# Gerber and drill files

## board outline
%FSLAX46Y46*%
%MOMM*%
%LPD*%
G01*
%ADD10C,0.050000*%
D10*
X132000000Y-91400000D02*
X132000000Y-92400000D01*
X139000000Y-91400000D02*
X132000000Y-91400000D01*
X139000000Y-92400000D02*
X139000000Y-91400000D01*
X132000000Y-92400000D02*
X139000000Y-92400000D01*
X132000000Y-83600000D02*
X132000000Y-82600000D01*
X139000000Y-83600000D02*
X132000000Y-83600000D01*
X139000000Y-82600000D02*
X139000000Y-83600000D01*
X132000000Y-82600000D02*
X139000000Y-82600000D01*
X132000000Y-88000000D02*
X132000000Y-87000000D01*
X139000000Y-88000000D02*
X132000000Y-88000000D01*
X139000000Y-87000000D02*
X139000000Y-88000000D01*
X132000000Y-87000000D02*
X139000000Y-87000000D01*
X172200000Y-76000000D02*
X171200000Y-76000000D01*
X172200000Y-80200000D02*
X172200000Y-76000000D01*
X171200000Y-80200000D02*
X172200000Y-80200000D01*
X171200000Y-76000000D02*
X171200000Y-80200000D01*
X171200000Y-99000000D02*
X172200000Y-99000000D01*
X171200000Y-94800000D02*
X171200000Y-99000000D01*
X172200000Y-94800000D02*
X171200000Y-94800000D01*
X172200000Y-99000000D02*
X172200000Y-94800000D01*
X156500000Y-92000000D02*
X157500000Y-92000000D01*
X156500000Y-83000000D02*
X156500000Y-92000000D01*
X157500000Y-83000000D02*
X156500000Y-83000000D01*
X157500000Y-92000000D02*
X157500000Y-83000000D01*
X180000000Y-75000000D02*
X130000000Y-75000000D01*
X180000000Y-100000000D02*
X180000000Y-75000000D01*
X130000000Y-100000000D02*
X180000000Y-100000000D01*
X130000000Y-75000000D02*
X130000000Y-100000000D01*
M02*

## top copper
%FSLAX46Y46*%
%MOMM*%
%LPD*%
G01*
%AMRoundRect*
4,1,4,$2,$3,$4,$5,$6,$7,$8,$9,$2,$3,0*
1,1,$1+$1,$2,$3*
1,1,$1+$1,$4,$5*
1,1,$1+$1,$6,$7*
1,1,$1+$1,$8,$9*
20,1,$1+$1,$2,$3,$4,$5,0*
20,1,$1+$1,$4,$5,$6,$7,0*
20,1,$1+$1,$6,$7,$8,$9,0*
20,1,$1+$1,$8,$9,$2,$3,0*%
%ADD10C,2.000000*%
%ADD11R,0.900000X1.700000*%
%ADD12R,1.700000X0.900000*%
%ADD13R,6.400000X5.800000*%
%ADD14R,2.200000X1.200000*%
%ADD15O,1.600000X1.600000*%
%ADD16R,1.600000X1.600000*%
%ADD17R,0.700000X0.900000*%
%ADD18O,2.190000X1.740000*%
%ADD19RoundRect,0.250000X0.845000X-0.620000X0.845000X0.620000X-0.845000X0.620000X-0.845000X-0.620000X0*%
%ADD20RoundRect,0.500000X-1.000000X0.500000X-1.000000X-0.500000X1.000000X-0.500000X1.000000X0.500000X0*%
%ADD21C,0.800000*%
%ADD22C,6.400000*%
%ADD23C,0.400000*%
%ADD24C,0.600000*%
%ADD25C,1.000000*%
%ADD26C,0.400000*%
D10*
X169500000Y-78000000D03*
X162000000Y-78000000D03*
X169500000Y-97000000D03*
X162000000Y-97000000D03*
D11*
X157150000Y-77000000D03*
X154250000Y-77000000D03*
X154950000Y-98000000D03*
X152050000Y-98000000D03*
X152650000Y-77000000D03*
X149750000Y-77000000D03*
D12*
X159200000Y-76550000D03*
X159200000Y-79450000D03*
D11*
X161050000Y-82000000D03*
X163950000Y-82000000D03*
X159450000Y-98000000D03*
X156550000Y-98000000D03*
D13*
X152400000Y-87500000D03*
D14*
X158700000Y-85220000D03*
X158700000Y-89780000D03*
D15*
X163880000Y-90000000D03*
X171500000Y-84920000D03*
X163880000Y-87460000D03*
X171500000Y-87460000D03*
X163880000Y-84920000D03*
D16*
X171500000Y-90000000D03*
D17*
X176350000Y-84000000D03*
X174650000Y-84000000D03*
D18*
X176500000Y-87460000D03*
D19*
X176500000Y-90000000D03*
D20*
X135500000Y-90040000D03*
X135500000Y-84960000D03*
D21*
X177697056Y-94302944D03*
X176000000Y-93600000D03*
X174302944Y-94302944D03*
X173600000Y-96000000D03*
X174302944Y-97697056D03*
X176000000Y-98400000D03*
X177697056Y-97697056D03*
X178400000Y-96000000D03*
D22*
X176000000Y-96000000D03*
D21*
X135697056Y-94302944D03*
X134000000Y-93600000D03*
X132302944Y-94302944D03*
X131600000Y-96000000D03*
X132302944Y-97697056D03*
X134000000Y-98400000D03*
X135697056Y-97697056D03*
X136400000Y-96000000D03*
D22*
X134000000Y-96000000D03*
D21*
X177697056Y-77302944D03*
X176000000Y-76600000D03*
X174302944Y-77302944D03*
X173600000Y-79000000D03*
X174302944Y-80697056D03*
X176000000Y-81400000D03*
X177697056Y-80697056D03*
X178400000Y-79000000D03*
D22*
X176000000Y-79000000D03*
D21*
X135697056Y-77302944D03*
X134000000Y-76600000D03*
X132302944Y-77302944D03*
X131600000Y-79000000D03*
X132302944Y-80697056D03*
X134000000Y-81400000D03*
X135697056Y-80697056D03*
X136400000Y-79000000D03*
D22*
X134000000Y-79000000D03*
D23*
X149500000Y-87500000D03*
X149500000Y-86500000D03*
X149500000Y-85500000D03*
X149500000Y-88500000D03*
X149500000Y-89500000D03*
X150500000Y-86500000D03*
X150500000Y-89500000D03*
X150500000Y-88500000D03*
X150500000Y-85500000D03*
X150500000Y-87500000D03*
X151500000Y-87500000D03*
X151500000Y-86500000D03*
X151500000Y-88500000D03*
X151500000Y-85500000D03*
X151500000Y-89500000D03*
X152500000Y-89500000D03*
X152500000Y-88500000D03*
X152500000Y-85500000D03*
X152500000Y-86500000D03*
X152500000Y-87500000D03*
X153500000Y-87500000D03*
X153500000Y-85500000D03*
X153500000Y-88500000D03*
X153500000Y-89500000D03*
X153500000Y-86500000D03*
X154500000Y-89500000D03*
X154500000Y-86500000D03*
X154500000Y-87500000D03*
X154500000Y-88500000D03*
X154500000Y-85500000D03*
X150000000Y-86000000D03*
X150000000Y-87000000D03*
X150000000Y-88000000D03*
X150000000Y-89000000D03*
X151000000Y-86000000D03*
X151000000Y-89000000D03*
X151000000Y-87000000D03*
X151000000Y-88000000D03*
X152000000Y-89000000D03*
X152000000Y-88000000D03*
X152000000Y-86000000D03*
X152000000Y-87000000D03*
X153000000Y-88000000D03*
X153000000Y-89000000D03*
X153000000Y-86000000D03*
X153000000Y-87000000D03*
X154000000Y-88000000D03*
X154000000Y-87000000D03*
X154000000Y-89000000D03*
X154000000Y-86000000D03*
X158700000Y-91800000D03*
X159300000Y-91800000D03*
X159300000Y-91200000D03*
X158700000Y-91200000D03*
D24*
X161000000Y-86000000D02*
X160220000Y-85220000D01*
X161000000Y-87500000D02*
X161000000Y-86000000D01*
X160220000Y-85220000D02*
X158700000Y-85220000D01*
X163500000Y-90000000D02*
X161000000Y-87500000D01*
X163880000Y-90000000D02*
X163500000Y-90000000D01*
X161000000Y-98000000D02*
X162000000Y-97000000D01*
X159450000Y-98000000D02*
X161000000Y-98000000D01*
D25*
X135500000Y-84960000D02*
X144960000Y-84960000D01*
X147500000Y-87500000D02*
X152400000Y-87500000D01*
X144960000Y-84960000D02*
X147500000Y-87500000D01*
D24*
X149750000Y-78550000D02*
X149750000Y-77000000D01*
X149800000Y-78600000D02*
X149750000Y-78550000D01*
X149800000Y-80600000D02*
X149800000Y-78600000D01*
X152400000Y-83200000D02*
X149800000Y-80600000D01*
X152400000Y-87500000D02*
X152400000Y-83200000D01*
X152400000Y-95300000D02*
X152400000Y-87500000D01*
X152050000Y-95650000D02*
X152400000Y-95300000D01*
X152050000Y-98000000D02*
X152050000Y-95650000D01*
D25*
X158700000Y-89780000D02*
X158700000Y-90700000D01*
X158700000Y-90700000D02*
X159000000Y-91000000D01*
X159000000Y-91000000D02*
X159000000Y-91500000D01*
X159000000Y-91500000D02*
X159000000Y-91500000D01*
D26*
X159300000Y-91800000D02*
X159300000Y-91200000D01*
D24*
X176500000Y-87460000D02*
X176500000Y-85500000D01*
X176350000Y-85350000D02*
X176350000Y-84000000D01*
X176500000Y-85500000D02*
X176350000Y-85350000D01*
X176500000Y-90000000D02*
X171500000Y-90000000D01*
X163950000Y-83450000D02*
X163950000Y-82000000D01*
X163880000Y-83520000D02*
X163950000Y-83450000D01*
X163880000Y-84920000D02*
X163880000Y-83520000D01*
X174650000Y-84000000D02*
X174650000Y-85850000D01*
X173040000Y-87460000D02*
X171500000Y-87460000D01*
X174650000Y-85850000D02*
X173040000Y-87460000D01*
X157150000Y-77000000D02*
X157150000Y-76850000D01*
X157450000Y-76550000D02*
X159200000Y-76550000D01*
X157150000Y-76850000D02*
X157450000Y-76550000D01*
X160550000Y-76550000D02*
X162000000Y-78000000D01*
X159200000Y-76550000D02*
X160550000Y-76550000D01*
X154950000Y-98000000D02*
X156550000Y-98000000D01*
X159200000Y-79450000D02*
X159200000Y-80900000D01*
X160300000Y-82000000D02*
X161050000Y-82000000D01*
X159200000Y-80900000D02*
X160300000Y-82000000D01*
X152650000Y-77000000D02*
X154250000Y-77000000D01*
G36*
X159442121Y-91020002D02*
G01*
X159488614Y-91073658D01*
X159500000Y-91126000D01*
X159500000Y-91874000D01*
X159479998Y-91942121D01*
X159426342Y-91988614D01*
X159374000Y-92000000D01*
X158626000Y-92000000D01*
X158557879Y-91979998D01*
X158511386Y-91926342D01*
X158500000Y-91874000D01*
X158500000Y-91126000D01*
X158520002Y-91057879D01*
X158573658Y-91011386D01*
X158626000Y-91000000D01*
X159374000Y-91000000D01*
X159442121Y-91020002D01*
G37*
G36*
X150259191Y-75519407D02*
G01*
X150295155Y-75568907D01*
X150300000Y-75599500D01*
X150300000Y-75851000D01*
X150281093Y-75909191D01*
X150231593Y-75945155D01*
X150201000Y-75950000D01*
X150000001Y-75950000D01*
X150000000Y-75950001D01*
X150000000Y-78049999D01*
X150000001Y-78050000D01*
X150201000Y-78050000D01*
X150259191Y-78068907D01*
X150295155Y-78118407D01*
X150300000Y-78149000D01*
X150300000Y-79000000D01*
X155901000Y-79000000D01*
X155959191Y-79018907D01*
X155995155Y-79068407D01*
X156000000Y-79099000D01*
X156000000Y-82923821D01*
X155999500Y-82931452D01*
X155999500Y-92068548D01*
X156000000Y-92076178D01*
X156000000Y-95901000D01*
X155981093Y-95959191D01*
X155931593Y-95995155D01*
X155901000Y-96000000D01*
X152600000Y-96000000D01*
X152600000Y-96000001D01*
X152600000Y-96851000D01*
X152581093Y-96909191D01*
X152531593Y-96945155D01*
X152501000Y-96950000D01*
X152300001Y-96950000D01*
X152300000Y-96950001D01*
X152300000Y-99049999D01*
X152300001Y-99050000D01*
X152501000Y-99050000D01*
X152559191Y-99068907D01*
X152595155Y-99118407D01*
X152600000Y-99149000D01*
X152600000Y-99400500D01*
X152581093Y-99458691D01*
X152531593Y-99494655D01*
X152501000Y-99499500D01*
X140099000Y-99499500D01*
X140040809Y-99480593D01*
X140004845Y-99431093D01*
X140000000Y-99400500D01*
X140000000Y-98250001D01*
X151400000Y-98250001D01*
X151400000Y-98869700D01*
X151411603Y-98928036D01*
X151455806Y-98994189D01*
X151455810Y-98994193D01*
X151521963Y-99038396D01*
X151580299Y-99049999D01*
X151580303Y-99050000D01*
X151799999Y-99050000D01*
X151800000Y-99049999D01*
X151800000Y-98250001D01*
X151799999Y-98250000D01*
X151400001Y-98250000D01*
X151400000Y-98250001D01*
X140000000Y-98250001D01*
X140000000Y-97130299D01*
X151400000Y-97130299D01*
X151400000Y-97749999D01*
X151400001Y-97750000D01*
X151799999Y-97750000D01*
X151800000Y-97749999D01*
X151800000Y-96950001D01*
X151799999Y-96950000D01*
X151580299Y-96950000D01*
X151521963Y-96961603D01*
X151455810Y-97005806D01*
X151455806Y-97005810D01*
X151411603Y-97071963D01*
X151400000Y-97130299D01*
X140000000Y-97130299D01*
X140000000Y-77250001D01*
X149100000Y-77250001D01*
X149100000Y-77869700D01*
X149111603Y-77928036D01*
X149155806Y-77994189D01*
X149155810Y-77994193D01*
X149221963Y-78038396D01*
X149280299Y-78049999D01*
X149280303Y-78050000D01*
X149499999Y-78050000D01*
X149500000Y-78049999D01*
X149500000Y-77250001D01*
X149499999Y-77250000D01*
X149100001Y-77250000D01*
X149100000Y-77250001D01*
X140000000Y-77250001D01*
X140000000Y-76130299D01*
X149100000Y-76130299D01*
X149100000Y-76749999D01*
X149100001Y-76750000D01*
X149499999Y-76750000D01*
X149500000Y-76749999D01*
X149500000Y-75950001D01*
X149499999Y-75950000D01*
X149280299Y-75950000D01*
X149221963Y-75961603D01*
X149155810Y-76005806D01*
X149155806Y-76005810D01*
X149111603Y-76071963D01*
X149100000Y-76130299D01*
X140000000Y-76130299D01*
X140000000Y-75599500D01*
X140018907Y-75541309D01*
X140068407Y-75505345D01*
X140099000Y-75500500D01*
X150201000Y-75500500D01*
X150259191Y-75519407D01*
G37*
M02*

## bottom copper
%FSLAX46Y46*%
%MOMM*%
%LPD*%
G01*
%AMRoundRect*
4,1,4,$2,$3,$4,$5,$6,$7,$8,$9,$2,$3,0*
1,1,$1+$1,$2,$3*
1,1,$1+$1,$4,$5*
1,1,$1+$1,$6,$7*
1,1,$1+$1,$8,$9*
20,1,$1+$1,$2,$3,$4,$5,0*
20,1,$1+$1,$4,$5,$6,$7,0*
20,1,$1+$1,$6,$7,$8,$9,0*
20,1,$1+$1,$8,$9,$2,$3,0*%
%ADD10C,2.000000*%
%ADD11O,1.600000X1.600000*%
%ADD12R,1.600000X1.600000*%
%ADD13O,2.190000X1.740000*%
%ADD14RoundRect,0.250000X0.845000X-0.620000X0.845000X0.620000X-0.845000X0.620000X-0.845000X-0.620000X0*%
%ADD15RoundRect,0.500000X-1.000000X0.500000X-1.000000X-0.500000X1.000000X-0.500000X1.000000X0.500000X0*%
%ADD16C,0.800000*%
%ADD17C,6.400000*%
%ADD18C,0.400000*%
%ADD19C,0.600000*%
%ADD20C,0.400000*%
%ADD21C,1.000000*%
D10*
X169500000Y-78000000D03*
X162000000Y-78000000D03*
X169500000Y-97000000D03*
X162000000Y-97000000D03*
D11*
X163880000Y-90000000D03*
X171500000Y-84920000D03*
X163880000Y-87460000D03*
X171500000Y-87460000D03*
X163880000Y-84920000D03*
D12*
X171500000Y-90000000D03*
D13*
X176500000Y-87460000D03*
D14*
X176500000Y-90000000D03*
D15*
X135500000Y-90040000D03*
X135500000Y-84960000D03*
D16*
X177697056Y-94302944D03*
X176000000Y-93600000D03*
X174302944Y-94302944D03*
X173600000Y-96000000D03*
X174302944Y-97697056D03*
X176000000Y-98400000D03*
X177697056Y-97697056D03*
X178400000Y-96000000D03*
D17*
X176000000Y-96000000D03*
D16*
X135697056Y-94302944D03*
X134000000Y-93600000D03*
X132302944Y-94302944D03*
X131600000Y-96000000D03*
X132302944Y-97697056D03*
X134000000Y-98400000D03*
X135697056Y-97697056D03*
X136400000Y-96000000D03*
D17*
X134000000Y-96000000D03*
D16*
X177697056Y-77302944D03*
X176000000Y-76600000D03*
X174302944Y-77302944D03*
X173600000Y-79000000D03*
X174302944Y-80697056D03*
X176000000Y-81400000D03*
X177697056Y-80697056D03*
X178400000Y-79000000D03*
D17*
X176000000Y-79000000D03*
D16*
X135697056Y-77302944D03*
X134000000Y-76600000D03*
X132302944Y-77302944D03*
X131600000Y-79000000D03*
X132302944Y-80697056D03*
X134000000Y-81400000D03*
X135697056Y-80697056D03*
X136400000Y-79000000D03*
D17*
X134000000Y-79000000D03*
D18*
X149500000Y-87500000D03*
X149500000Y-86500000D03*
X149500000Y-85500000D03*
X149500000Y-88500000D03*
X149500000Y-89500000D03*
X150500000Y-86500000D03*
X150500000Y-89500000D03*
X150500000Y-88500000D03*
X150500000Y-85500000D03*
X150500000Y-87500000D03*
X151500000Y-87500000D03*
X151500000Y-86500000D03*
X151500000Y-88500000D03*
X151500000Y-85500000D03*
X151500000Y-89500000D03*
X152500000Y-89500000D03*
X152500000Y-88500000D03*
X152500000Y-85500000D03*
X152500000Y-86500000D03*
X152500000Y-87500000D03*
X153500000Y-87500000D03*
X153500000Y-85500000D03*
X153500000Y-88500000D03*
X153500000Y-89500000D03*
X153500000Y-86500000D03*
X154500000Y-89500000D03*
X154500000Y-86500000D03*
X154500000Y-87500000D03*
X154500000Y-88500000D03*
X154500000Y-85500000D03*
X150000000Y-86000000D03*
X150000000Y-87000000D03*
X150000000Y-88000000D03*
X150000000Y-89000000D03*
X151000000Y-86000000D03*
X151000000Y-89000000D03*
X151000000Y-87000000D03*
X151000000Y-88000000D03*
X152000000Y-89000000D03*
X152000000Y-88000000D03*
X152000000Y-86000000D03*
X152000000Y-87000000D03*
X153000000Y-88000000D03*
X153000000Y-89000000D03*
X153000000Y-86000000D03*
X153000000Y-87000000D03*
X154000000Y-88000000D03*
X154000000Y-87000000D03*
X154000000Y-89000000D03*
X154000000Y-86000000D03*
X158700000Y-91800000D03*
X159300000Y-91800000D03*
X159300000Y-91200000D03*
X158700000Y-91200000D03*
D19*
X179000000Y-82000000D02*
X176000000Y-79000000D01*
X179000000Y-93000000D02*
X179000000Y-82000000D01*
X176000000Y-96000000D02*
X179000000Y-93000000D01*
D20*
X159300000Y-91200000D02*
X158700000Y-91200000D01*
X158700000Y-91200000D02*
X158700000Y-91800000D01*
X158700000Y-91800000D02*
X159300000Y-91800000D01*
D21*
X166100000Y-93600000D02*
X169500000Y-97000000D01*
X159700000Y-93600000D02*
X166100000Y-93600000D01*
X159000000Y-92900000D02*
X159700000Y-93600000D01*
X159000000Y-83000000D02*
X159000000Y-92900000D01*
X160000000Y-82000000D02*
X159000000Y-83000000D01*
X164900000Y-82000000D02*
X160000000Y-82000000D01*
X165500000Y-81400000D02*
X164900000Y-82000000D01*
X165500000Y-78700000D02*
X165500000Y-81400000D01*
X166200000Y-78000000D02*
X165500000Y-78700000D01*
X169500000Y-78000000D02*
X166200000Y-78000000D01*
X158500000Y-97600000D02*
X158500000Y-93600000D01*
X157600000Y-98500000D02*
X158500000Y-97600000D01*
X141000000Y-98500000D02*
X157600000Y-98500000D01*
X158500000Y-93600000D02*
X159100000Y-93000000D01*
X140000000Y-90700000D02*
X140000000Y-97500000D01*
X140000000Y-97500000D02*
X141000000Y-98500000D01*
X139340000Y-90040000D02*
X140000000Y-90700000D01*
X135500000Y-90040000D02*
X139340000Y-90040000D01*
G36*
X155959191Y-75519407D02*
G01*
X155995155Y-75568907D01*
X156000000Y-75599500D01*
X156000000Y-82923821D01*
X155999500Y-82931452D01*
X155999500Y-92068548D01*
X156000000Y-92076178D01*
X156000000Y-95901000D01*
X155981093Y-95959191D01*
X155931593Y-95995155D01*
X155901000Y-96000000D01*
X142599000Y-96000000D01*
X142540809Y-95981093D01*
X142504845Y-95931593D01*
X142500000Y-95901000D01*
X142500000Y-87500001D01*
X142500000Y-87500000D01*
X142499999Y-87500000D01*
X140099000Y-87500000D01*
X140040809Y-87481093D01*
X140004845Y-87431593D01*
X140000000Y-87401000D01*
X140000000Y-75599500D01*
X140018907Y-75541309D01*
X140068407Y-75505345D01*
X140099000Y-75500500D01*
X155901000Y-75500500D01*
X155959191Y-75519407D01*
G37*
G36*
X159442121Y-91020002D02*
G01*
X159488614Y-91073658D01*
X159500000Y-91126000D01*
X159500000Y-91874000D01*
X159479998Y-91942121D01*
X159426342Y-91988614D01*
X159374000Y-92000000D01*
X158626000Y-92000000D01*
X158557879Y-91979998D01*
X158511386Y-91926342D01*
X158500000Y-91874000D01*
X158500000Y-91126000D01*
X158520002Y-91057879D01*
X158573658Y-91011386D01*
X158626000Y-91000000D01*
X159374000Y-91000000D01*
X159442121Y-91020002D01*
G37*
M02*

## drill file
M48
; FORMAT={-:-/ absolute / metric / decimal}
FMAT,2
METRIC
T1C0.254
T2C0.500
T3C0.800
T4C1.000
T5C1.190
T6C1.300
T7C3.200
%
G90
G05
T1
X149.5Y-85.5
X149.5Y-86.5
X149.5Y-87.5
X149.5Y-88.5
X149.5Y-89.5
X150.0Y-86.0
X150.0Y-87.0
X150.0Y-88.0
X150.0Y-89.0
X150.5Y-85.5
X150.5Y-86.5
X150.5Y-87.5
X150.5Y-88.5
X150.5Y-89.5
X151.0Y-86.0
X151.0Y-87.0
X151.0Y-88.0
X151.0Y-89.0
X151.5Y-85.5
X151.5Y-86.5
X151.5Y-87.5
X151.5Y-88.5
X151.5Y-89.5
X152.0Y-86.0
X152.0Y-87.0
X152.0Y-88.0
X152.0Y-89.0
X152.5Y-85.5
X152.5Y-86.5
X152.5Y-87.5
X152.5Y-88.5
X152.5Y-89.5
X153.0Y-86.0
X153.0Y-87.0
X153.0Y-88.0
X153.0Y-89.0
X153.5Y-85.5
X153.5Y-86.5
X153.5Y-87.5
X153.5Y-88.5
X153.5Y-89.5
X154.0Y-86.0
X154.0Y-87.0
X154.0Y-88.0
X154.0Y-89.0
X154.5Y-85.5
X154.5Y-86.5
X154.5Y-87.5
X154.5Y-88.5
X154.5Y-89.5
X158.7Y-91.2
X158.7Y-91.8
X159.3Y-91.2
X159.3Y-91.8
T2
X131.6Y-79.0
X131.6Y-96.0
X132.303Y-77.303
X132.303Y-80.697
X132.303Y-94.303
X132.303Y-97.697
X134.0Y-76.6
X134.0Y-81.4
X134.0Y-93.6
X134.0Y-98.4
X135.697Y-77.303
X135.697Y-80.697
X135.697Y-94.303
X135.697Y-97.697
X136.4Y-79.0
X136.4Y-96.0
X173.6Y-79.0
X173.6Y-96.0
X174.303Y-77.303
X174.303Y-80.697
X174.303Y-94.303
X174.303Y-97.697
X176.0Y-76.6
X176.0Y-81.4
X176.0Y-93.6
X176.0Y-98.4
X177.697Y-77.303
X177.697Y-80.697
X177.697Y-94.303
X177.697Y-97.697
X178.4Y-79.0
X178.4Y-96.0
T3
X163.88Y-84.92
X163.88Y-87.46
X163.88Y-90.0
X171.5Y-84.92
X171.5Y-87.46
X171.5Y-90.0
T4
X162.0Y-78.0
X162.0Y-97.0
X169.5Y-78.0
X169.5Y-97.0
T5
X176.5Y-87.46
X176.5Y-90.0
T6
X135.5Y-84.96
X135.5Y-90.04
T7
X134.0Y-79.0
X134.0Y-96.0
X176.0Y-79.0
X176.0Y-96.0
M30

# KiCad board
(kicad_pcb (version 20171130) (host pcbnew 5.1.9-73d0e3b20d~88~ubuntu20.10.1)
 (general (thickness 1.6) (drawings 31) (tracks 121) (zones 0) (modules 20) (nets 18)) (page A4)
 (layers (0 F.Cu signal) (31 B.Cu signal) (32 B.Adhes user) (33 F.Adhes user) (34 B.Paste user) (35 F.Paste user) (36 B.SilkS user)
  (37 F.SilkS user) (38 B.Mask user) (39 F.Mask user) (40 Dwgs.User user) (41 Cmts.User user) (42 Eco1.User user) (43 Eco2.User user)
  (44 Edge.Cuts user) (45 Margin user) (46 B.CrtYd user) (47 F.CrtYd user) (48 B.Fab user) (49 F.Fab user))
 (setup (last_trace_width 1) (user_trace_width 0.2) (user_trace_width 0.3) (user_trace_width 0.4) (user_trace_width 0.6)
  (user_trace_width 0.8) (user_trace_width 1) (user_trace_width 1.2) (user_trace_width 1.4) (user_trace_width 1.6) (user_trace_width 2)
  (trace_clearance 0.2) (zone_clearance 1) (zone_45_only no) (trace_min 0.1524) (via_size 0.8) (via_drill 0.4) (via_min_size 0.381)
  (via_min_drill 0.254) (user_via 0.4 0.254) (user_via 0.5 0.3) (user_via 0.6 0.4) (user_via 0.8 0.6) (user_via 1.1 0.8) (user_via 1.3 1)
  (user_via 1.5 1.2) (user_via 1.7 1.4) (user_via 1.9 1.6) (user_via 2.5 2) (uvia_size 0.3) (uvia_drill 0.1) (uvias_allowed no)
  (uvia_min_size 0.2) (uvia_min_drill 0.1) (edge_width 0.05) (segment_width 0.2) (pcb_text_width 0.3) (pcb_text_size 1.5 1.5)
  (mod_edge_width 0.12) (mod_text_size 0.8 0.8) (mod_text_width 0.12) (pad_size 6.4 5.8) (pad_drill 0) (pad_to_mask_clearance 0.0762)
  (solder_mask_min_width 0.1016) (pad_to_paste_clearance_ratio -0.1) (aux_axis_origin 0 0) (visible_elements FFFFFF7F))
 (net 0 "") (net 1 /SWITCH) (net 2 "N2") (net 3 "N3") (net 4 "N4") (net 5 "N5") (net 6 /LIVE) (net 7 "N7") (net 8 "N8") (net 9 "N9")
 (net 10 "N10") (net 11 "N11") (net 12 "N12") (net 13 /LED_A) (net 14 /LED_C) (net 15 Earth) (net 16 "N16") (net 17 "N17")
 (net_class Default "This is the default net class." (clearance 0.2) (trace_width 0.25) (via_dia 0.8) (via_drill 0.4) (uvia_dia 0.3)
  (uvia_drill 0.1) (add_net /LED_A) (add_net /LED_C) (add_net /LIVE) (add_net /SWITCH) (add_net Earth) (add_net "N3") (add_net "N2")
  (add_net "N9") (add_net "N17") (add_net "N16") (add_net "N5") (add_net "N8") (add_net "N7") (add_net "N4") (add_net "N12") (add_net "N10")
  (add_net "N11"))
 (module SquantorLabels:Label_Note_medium (layer F.Cu) (at 145.3 87.4 90)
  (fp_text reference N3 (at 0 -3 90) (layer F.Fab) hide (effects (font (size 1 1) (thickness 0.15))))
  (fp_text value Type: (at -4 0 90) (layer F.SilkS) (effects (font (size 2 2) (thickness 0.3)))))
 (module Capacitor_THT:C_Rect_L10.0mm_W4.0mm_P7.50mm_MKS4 (layer F.Cu) (at 162 78)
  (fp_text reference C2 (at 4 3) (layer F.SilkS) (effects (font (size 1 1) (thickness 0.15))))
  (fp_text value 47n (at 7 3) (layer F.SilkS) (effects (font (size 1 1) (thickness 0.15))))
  (pad 2 thru_hole circle (at 7.5 0) (size 2 2) (drill 1) (layers *.Cu *.Mask) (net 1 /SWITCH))
  (pad 1 thru_hole circle (at 0 0) (size 2 2) (drill 1) (layers *.Cu *.Mask) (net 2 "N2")))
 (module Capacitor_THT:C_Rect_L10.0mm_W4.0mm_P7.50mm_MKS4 (layer F.Cu) (at 162 97)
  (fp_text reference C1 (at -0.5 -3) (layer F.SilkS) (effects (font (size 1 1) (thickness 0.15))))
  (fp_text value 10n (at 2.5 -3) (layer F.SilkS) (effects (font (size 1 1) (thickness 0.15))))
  (pad 2 thru_hole circle (at 7.5 0) (size 2 2) (drill 1) (layers *.Cu *.Mask) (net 1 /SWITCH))
  (pad 1 thru_hole circle (at 0 0) (size 2 2) (drill 1) (layers *.Cu *.Mask) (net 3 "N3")))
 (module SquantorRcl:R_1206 (layer F.Cu) (at 155.7 77)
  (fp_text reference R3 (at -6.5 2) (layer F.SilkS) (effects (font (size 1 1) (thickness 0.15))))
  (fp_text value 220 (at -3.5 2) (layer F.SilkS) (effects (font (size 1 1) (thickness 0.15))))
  (pad 2 smd rect (at 1.45 0) (size 0.9 1.7) (layers F.Cu F.Paste F.Mask) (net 2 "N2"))
  (pad 1 smd rect (at -1.45 0) (size 0.9 1.7) (layers F.Cu F.Paste F.Mask) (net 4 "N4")))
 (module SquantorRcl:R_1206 (layer F.Cu) (at 153.5 98)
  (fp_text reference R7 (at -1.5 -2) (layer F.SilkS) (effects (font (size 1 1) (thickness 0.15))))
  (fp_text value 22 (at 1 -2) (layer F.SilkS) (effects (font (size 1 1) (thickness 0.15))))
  (pad 2 smd rect (at 1.45 0) (size 0.9 1.7) (layers F.Cu F.Paste F.Mask) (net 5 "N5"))
  (pad 1 smd rect (at -1.45 0) (size 0.9 1.7) (layers F.Cu F.Paste F.Mask) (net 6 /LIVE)))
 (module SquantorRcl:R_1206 (layer F.Cu) (at 151.2 77)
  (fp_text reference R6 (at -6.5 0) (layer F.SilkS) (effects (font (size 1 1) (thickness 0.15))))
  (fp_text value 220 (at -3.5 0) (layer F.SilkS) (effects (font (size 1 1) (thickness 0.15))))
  (pad 2 smd rect (at 1.45 0) (size 0.9 1.7) (layers F.Cu F.Paste F.Mask) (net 4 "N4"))
  (pad 1 smd rect (at -1.45 0) (size 0.9 1.7) (layers F.Cu F.Paste F.Mask) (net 6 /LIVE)))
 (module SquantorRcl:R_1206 (layer F.Cu) (at 159.2 78 90)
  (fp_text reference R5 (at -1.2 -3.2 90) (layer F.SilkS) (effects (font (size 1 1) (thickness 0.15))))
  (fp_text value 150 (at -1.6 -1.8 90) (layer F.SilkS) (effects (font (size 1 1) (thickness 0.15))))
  (pad 2 smd rect (at 1.45 0 90) (size 0.9 1.7) (layers F.Cu F.Paste F.Mask) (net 2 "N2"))
  (pad 1 smd rect (at -1.45 0 90) (size 0.9 1.7) (layers F.Cu F.Paste F.Mask) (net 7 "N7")))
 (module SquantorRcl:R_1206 (layer F.Cu) (at 162.5 82 180)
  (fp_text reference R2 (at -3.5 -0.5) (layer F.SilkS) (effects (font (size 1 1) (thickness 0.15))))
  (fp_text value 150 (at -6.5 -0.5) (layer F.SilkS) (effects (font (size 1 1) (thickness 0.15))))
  (pad 2 smd rect (at 1.45 0 180) (size 0.9 1.7) (layers F.Cu F.Paste F.Mask) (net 7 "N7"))
  (pad 1 smd rect (at -1.45 0 180) (size 0.9 1.7) (layers F.Cu F.Paste F.Mask) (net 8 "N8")))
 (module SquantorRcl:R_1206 (layer F.Cu) (at 158 98)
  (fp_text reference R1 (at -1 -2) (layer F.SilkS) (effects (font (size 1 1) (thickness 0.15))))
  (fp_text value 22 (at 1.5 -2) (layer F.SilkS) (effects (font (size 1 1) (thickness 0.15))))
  (pad 2 smd rect (at 1.45 0) (size 0.9 1.7) (layers F.Cu F.Paste F.Mask) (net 3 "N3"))
  (pad 1 smd rect (at -1.45 0) (size 0.9 1.7) (layers F.Cu F.Paste F.Mask) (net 5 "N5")))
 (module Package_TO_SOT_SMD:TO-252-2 (layer F.Cu) (at 154.5 87.5 180)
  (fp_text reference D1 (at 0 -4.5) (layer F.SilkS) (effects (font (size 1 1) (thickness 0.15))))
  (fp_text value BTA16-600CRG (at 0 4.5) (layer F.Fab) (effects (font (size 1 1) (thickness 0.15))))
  (pad "" smd rect (at 0.425 1.525 180) (size 3.05 2.75) (layers F.Paste))
  (pad "" smd rect (at 3.775 -1.525 180) (size 3.05 2.75) (layers F.Paste))
  (pad "" smd rect (at 0.425 -1.525 180) (size 3.05 2.75) (layers F.Paste))
  (pad "" smd rect (at 3.775 1.525 180) (size 3.05 2.75) (layers F.Paste))
  (pad 2 smd rect (at 2.1 0 180) (size 6.4 5.8) (layers F.Cu F.Mask) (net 6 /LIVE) (zone_connect 2))
  (pad 3 smd rect (at -4.2 2.28 180) (size 2.2 1.2) (layers F.Cu F.Paste F.Mask) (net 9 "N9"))
  (pad 1 smd rect (at -4.2 -2.28 180) (size 2.2 1.2) (layers F.Cu F.Paste F.Mask) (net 1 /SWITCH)))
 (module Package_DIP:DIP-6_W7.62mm (layer F.Cu) (at 171.5 90 180)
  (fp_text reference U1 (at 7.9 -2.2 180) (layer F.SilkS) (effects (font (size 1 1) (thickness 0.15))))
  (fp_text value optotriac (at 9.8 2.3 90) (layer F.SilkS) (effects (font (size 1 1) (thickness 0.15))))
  (pad 6 thru_hole oval (at 7.62 0 180) (size 1.6 1.6) (drill 0.8) (layers *.Cu *.Mask) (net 9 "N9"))
  (pad 3 thru_hole oval (at 0 5.08 180) (size 1.6 1.6) (drill 0.8) (layers *.Cu *.Mask) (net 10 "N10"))
  (pad 5 thru_hole oval (at 7.62 2.54 180) (size 1.6 1.6) (drill 0.8) (layers *.Cu *.Mask) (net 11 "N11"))
  (pad 2 thru_hole oval (at 0 2.54 180) (size 1.6 1.6) (drill 0.8) (layers *.Cu *.Mask) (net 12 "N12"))
  (pad 4 thru_hole oval (at 7.62 5.08 180) (size 1.6 1.6) (drill 0.8) (layers *.Cu *.Mask) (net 8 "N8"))
  (pad 1 thru_hole rect (at 0 0 180) (size 1.6 1.6) (drill 0.8) (layers *.Cu *.Mask) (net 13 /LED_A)))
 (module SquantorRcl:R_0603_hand (layer F.Cu) (at 175.5 84)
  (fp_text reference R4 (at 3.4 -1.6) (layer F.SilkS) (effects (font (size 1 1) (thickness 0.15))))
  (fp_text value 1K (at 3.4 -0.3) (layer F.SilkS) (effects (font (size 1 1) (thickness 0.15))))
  (pad 2 smd rect (at 0.85 0) (size 0.7 0.9) (layers F.Cu F.Paste F.Mask) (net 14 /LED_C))
  (pad 1 smd rect (at -0.85 0) (size 0.7 0.9) (layers F.Cu F.Paste F.Mask) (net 12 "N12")))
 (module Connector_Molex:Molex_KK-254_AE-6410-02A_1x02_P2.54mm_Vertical (layer F.Cu) (at 176.5 90 90)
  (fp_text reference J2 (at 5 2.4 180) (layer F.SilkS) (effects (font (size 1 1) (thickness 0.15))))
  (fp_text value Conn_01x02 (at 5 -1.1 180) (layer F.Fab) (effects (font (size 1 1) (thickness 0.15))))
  (pad 2 thru_hole oval (at 2.54 0 90) (size 1.74 2.19) (drill 1.19) (layers *.Cu *.Mask) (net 14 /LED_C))
  (pad 1 thru_hole roundrect (at 0 0 90) (size 1.74 2.19) (drill 1.19) (layers *.Cu *.Mask) (roundrect_rratio 0.143678) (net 13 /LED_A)))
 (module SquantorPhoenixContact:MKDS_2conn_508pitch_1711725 (layer F.Cu) (at 135.5 87.5 270)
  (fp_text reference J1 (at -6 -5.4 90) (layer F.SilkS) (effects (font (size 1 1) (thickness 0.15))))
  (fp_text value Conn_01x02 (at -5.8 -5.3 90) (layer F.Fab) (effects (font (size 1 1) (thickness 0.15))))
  (pad 2 thru_hole roundrect (at 2.54 0 270) (size 2 3) (drill 1.3) (layers *.Cu *.Mask) (roundrect_rratio 0.25) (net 1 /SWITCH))
  (pad 1 thru_hole roundrect (at -2.54 0 270) (size 2 3) (drill 1.3) (layers *.Cu *.Mask) (roundrect_rratio 0.25) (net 6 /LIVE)))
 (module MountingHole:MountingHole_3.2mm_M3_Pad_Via (layer F.Cu) (at 176 96)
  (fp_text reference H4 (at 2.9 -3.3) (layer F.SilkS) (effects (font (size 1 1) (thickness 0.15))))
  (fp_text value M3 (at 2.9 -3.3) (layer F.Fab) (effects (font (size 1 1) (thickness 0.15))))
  (pad 1 thru_hole circle (at 1.697056 -1.697056) (size 0.8 0.8) (drill 0.5) (layers *.Cu *.Mask) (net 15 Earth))
  (pad 1 thru_hole circle (at 0 -2.4) (size 0.8 0.8) (drill 0.5) (layers *.Cu *.Mask) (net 15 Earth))
  (pad 1 thru_hole circle (at -1.697056 -1.697056) (size 0.8 0.8) (drill 0.5) (layers *.Cu *.Mask) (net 15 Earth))
  (pad 1 thru_hole circle (at -2.4 0) (size 0.8 0.8) (drill 0.5) (layers *.Cu *.Mask) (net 15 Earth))
  (pad 1 thru_hole circle (at -1.697056 1.697056) (size 0.8 0.8) (drill 0.5) (layers *.Cu *.Mask) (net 15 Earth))
  (pad 1 thru_hole circle (at 0 2.4) (size 0.8 0.8) (drill 0.5) (layers *.Cu *.Mask) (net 15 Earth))
  (pad 1 thru_hole circle (at 1.697056 1.697056) (size 0.8 0.8) (drill 0.5) (layers *.Cu *.Mask) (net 15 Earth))
  (pad 1 thru_hole circle (at 2.4 0) (size 0.8 0.8) (drill 0.5) (layers *.Cu *.Mask) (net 15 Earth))
  (pad 1 thru_hole circle (at 0 0) (size 6.4 6.4) (drill 3.2) (layers *.Cu *.Mask) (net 15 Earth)))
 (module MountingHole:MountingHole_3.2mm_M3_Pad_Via (layer F.Cu) (at 134 96)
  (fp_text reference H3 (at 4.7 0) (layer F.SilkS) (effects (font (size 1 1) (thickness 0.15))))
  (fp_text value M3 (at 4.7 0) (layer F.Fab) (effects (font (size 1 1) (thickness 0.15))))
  (pad 1 thru_hole circle (at 1.697056 -1.697056) (size 0.8 0.8) (drill 0.5) (layers *.Cu *.Mask) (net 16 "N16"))
  (pad 1 thru_hole circle (at 0 -2.4) (size 0.8 0.8) (drill 0.5) (layers *.Cu *.Mask) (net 16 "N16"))
  (pad 1 thru_hole circle (at -1.697056 -1.697056) (size 0.8 0.8) (drill 0.5) (layers *.Cu *.Mask) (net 16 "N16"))
  (pad 1 thru_hole circle (at -2.4 0) (size 0.8 0.8) (drill 0.5) (layers *.Cu *.Mask) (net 16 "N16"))
  (pad 1 thru_hole circle (at -1.697056 1.697056) (size 0.8 0.8) (drill 0.5) (layers *.Cu *.Mask) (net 16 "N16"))
  (pad 1 thru_hole circle (at 0 2.4) (size 0.8 0.8) (drill 0.5) (layers *.Cu *.Mask) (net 16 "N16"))
  (pad 1 thru_hole circle (at 1.697056 1.697056) (size 0.8 0.8) (drill 0.5) (layers *.Cu *.Mask) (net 16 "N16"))
  (pad 1 thru_hole circle (at 2.4 0) (size 0.8 0.8) (drill 0.5) (layers *.Cu *.Mask) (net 16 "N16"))
  (pad 1 thru_hole circle (at 0 0) (size 6.4 6.4) (drill 3.2) (layers *.Cu *.Mask) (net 16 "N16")))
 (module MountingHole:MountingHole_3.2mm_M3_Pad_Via (layer F.Cu) (at 176 79)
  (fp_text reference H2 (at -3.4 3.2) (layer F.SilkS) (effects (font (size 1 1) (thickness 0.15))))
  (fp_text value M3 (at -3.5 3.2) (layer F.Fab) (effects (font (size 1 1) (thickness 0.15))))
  (pad 1 thru_hole circle (at 1.697056 -1.697056) (size 0.8 0.8) (drill 0.5) (layers *.Cu *.Mask) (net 15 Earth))
  (pad 1 thru_hole circle (at 0 -2.4) (size 0.8 0.8) (drill 0.5) (layers *.Cu *.Mask) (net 15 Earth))
  (pad 1 thru_hole circle (at -1.697056 -1.697056) (size 0.8 0.8) (drill 0.5) (layers *.Cu *.Mask) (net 15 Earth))
  (pad 1 thru_hole circle (at -2.4 0) (size 0.8 0.8) (drill 0.5) (layers *.Cu *.Mask) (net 15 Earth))
  (pad 1 thru_hole circle (at -1.697056 1.697056) (size 0.8 0.8) (drill 0.5) (layers *.Cu *.Mask) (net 15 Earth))
  (pad 1 thru_hole circle (at 0 2.4) (size 0.8 0.8) (drill 0.5) (layers *.Cu *.Mask) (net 15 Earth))
  (pad 1 thru_hole circle (at 1.697056 1.697056) (size 0.8 0.8) (drill 0.5) (layers *.Cu *.Mask) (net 15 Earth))
  (pad 1 thru_hole circle (at 2.4 0) (size 0.8 0.8) (drill 0.5) (layers *.Cu *.Mask) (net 15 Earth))
  (pad 1 thru_hole circle (at 0 0) (size 6.4 6.4) (drill 3.2) (layers *.Cu *.Mask) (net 15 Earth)))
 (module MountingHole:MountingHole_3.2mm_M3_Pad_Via (layer F.Cu) (at 134 79)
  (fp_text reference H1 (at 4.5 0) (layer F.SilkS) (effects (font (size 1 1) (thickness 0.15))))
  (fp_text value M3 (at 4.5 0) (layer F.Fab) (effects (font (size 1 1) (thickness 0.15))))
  (pad 1 thru_hole circle (at 1.697056 -1.697056) (size 0.8 0.8) (drill 0.5) (layers *.Cu *.Mask) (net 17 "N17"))
  (pad 1 thru_hole circle (at 0 -2.4) (size 0.8 0.8) (drill 0.5) (layers *.Cu *.Mask) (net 17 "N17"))
  (pad 1 thru_hole circle (at -1.697056 -1.697056) (size 0.8 0.8) (drill 0.5) (layers *.Cu *.Mask) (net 17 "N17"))
  (pad 1 thru_hole circle (at -2.4 0) (size 0.8 0.8) (drill 0.5) (layers *.Cu *.Mask) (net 17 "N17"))
  (pad 1 thru_hole circle (at -1.697056 1.697056) (size 0.8 0.8) (drill 0.5) (layers *.Cu *.Mask) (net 17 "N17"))
  (pad 1 thru_hole circle (at 0 2.4) (size 0.8 0.8) (drill 0.5) (layers *.Cu *.Mask) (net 17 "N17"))
  (pad 1 thru_hole circle (at 1.697056 1.697056) (size 0.8 0.8) (drill 0.5) (layers *.Cu *.Mask) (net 17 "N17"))
  (pad 1 thru_hole circle (at 2.4 0) (size 0.8 0.8) (drill 0.5) (layers *.Cu *.Mask) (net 17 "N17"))
  (pad 1 thru_hole circle (at 0 0) (size 6.4 6.4) (drill 3.2) (layers *.Cu *.Mask) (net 17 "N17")))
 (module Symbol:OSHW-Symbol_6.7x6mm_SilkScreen (layer B.Cu) (at 143.6 87.5 270)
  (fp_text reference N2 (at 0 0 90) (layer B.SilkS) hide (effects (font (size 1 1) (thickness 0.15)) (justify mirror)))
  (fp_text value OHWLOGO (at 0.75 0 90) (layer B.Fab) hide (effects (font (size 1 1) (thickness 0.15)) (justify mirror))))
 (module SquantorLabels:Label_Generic (layer B.Cu) (at 147.5 86.9 270)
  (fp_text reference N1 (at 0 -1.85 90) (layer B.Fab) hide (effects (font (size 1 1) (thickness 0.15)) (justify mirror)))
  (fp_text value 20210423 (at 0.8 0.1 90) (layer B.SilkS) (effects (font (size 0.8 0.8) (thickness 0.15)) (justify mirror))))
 (gr_line (start 132 91.4) (end 132 92.4) (layer Edge.Cuts) (width 0.05))
 (gr_line (start 139 91.4) (end 132 91.4) (layer Edge.Cuts) (width 0.05))
 (gr_line (start 139 92.4) (end 139 91.4) (layer Edge.Cuts) (width 0.05))
 (gr_line (start 132 92.4) (end 139 92.4) (layer Edge.Cuts) (width 0.05))
 (gr_line (start 132 83.6) (end 132 82.6) (layer Edge.Cuts) (width 0.05))
 (gr_line (start 139 83.6) (end 132 83.6) (layer Edge.Cuts) (width 0.05))
 (gr_line (start 139 82.6) (end 139 83.6) (layer Edge.Cuts) (width 0.05))
 (gr_line (start 132 82.6) (end 139 82.6) (layer Edge.Cuts) (width 0.05))
 (gr_line (start 132 88) (end 132 87) (layer Edge.Cuts) (width 0.05))
 (gr_line (start 139 88) (end 132 88) (layer Edge.Cuts) (width 0.05))
 (gr_line (start 139 87) (end 139 88) (layer Edge.Cuts) (width 0.05))
 (gr_line (start 132 87) (end 139 87) (layer Edge.Cuts) (width 0.05))
 (gr_line (start 172.2 76) (end 171.2 76) (layer Edge.Cuts) (width 0.05))
 (gr_line (start 172.2 80.2) (end 172.2 76) (layer Edge.Cuts) (width 0.05))
 (gr_line (start 171.2 80.2) (end 172.2 80.2) (layer Edge.Cuts) (width 0.05))
 (gr_line (start 171.2 76) (end 171.2 80.2) (layer Edge.Cuts) (width 0.05))
 (gr_line (start 171.2 99) (end 172.2 99) (layer Edge.Cuts) (width 0.05))
 (gr_line (start 171.2 94.8) (end 171.2 99) (layer Edge.Cuts) (width 0.05))
 (gr_line (start 172.2 94.8) (end 171.2 94.8) (layer Edge.Cuts) (width 0.05))
 (gr_line (start 172.2 99) (end 172.2 94.8) (layer Edge.Cuts) (width 0.05))
 (gr_line (start 156.5 92) (end 157.5 92) (layer Edge.Cuts) (width 0.05))
 (gr_line (start 156.5 83) (end 156.5 92) (layer Edge.Cuts) (width 0.05))
 (gr_line (start 157.5 83) (end 156.5 83) (layer Edge.Cuts) (width 0.05))
 (gr_line (start 157.5 92) (end 157.5 83) (layer Edge.Cuts) (width 0.05))
 (gr_line (start 180 75) (end 130 75) (layer Edge.Cuts) (width 0.05))
 (gr_line (start 180 100) (end 180 75) (layer Edge.Cuts) (width 0.05))
 (gr_line (start 130 100) (end 180 100) (layer Edge.Cuts) (width 0.05))
 (gr_line (start 130 75) (end 130 100) (layer Edge.Cuts) (width 0.05))
 (segment (start 161 86) (end 160.22 85.22) (width 0.6) (layer F.Cu) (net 9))
 (segment (start 161 87.5) (end 161 86) (width 0.6) (layer F.Cu) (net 9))
 (segment (start 160.22 85.22) (end 158.7 85.22) (width 0.6) (layer F.Cu) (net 9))
 (segment (start 163.5 90) (end 161 87.5) (width 0.6) (layer F.Cu) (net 9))
 (segment (start 163.88 90) (end 163.5 90) (width 0.6) (layer F.Cu) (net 9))
 (segment (start 179 82) (end 176 79) (width 0.6) (layer B.Cu) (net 15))
 (segment (start 179 93) (end 179 82) (width 0.6) (layer B.Cu) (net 15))
 (segment (start 176 96) (end 179 93) (width 0.6) (layer B.Cu) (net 15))
 (segment (start 161 98) (end 162 97) (width 0.6) (layer F.Cu) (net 3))
 (segment (start 159.45 98) (end 161 98) (width 0.6) (layer F.Cu) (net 3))
 (segment (start 135.5 84.96) (end 144.96 84.96) (width 1) (layer F.Cu) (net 6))
 (segment (start 147.5 87.5) (end 152.4 87.5) (width 1) (layer F.Cu) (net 6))
 (segment (start 144.96 84.96) (end 147.5 87.5) (width 1) (layer F.Cu) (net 6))
 (via (at 149.5 87.5) (size 0.4) (drill 0.254) (layers F.Cu B.Cu) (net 6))
 (via (at 149.5 86.5) (size 0.4) (drill 0.254) (layers F.Cu B.Cu) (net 6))
 (via (at 149.5 85.5) (size 0.4) (drill 0.254) (layers F.Cu B.Cu) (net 6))
 (via (at 149.5 88.5) (size 0.4) (drill 0.254) (layers F.Cu B.Cu) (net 6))
 (via (at 149.5 89.5) (size 0.4) (drill 0.254) (layers F.Cu B.Cu) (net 6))
 (via (at 150.5 86.5) (size 0.4) (drill 0.254) (layers F.Cu B.Cu) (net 6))
 (via (at 150.5 89.5) (size 0.4) (drill 0.254) (layers F.Cu B.Cu) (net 6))
 (via (at 150.5 88.5) (size 0.4) (drill 0.254) (layers F.Cu B.Cu) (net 6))
 (via (at 150.5 85.5) (size 0.4) (drill 0.254) (layers F.Cu B.Cu) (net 6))
 (via (at 150.5 87.5) (size 0.4) (drill 0.254) (layers F.Cu B.Cu) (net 6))
 (via (at 151.5 87.5) (size 0.4) (drill 0.254) (layers F.Cu B.Cu) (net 6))
 (via (at 151.5 86.5) (size 0.4) (drill 0.254) (layers F.Cu B.Cu) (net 6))
 (via (at 151.5 88.5) (size 0.4) (drill 0.254) (layers F.Cu B.Cu) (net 6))
 (via (at 151.5 85.5) (size 0.4) (drill 0.254) (layers F.Cu B.Cu) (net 6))
 (via (at 151.5 89.5) (size 0.4) (drill 0.254) (layers F.Cu B.Cu) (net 6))
 (via (at 152.5 89.5) (size 0.4) (drill 0.254) (layers F.Cu B.Cu) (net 6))
 (via (at 152.5 88.5) (size 0.4) (drill 0.254) (layers F.Cu B.Cu) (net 6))
 (via (at 152.5 85.5) (size 0.4) (drill 0.254) (layers F.Cu B.Cu) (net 6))
 (via (at 152.5 86.5) (size 0.4) (drill 0.254) (layers F.Cu B.Cu) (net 6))
 (via (at 152.5 87.5) (size 0.4) (drill 0.254) (layers F.Cu B.Cu) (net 6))
 (via (at 153.5 87.5) (size 0.4) (drill 0.254) (layers F.Cu B.Cu) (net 6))
 (via (at 153.5 85.5) (size 0.4) (drill 0.254) (layers F.Cu B.Cu) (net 6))
 (via (at 153.5 88.5) (size 0.4) (drill 0.254) (layers F.Cu B.Cu) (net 6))
 (via (at 153.5 89.5) (size 0.4) (drill 0.254) (layers F.Cu B.Cu) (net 6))
 (via (at 153.5 86.5) (size 0.4) (drill 0.254) (layers F.Cu B.Cu) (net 6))
 (via (at 154.5 89.5) (size 0.4) (drill 0.254) (layers F.Cu B.Cu) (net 6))
 (via (at 154.5 86.5) (size 0.4) (drill 0.254) (layers F.Cu B.Cu) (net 6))
 (via (at 154.5 87.5) (size 0.4) (drill 0.254) (layers F.Cu B.Cu) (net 6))
 (via (at 154.5 88.5) (size 0.4) (drill 0.254) (layers F.Cu B.Cu) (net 6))
 (via (at 154.5 85.5) (size 0.4) (drill 0.254) (layers F.Cu B.Cu) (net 6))
 (via (at 150 86) (size 0.4) (drill 0.254) (layers F.Cu B.Cu) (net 6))
 (via (at 150 87) (size 0.4) (drill 0.254) (layers F.Cu B.Cu) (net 6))
 (via (at 150 88) (size 0.4) (drill 0.254) (layers F.Cu B.Cu) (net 6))
 (via (at 150 89) (size 0.4) (drill 0.254) (layers F.Cu B.Cu) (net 6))
 (via (at 151 86) (size 0.4) (drill 0.254) (layers F.Cu B.Cu) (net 6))
 (via (at 151 89) (size 0.4) (drill 0.254) (layers F.Cu B.Cu) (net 6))
 (via (at 151 87) (size 0.4) (drill 0.254) (layers F.Cu B.Cu) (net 6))
 (via (at 151 88) (size 0.4) (drill 0.254) (layers F.Cu B.Cu) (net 6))
 (via (at 152 89) (size 0.4) (drill 0.254) (layers F.Cu B.Cu) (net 6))
 (via (at 152 88) (size 0.4) (drill 0.254) (layers F.Cu B.Cu) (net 6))
 (via (at 152 86) (size 0.4) (drill 0.254) (layers F.Cu B.Cu) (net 6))
 (via (at 152 87) (size 0.4) (drill 0.254) (layers F.Cu B.Cu) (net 6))
 (via (at 153 88) (size 0.4) (drill 0.254) (layers F.Cu B.Cu) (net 6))
 (via (at 153 89) (size 0.4) (drill 0.254) (layers F.Cu B.Cu) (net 6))
 (via (at 153 86) (size 0.4) (drill 0.254) (layers F.Cu B.Cu) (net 6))
 (via (at 153 87) (size 0.4) (drill 0.254) (layers F.Cu B.Cu) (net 6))
 (via (at 154 88) (size 0.4) (drill 0.254) (layers F.Cu B.Cu) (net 6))
 (via (at 154 87) (size 0.4) (drill 0.254) (layers F.Cu B.Cu) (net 6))
 (via (at 154 89) (size 0.4) (drill 0.254) (layers F.Cu B.Cu) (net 6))
 (via (at 154 86) (size 0.4) (drill 0.254) (layers F.Cu B.Cu) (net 6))
 (segment (start 149.75 78.55) (end 149.75 77) (width 0.6) (layer F.Cu) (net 6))
 (segment (start 149.8 78.6) (end 149.75 78.55) (width 0.6) (layer F.Cu) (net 6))
 (segment (start 149.8 80.6) (end 149.8 78.6) (width 0.6) (layer F.Cu) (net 6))
 (segment (start 152.4 83.2) (end 149.8 80.6) (width 0.6) (layer F.Cu) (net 6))
 (segment (start 152.4 87.5) (end 152.4 83.2) (width 0.6) (layer F.Cu) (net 6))
 (segment (start 152.4 95.3) (end 152.4 87.5) (width 0.6) (layer F.Cu) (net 6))
 (segment (start 152.05 95.65) (end 152.4 95.3) (width 0.6) (layer F.Cu) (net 6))
 (segment (start 152.05 98) (end 152.05 95.65) (width 0.6) (layer F.Cu) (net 6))
 (segment (start 158.7 89.78) (end 158.7 90.7) (width 1) (layer F.Cu) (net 1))
 (segment (start 158.7 90.7) (end 159 91) (width 1) (layer F.Cu) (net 1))
 (segment (start 159 91) (end 159 91.5) (width 1) (layer F.Cu) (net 1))
 (segment (start 159 91.5) (end 159 91.5) (width 1) (layer F.Cu) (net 1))
 (via (at 158.7 91.8) (size 0.4) (drill 0.254) (layers F.Cu B.Cu) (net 1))
 (via (at 159.3 91.8) (size 0.4) (drill 0.254) (layers F.Cu B.Cu) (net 1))
 (via (at 159.3 91.2) (size 0.4) (drill 0.254) (layers F.Cu B.Cu) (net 1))
 (via (at 158.7 91.2) (size 0.4) (drill 0.254) (layers F.Cu B.Cu) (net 1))
 (segment (start 159.3 91.8) (end 159.3 91.2) (width 0.4) (layer F.Cu) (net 1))
 (segment (start 159.3 91.2) (end 158.7 91.2) (width 0.4) (layer B.Cu) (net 1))
 (segment (start 158.7 91.2) (end 158.7 91.8) (width 0.4) (layer B.Cu) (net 1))
 (segment (start 158.7 91.8) (end 159.3 91.8) (width 0.4) (layer B.Cu) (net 1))
 (segment (start 166.1 93.6) (end 169.5 97) (width 1) (layer B.Cu) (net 1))
 (segment (start 159.7 93.6) (end 166.1 93.6) (width 1) (layer B.Cu) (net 1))
 (segment (start 159 92.9) (end 159.7 93.6) (width 1) (layer B.Cu) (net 1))
 (segment (start 159 83) (end 159 92.9) (width 1) (layer B.Cu) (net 1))
 (segment (start 160 82) (end 159 83) (width 1) (layer B.Cu) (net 1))
 (segment (start 164.9 82) (end 160 82) (width 1) (layer B.Cu) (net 1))
 (segment (start 165.5 81.4) (end 164.9 82) (width 1) (layer B.Cu) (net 1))
 (segment (start 165.5 78.7) (end 165.5 81.4) (width 1) (layer B.Cu) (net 1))
 (segment (start 166.2 78) (end 165.5 78.7) (width 1) (layer B.Cu) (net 1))
 (segment (start 169.5 78) (end 166.2 78) (width 1) (layer B.Cu) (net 1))
 (segment (start 158.5 97.6) (end 158.5 93.6) (width 1) (layer B.Cu) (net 1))
 (segment (start 157.6 98.5) (end 158.5 97.6) (width 1) (layer B.Cu) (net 1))
 (segment (start 141 98.5) (end 157.6 98.5) (width 1) (layer B.Cu) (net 1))
 (segment (start 158.5 93.6) (end 159.1 93) (width 1) (layer B.Cu) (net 1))
 (segment (start 140 90.7) (end 140 97.5) (width 1) (layer B.Cu) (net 1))
 (segment (start 140 97.5) (end 141 98.5) (width 1) (layer B.Cu) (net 1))
 (segment (start 139.34 90.04) (end 140 90.7) (width 1) (layer B.Cu) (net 1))
 (segment (start 135.5 90.04) (end 139.34 90.04) (width 1) (layer B.Cu) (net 1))
 (segment (start 176.5 87.46) (end 176.5 85.5) (width 0.6) (layer F.Cu) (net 14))
 (segment (start 176.35 85.35) (end 176.35 84) (width 0.6) (layer F.Cu) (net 14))
 (segment (start 176.5 85.5) (end 176.35 85.35) (width 0.6) (layer F.Cu) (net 14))
 (segment (start 176.5 90) (end 171.5 90) (width 0.6) (layer F.Cu) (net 13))
 (segment (start 163.95 83.45) (end 163.95 82) (width 0.6) (layer F.Cu) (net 8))
 (segment (start 163.88 83.52) (end 163.95 83.45) (width 0.6) (layer F.Cu) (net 8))
 (segment (start 163.88 84.92) (end 163.88 83.52) (width 0.6) (layer F.Cu) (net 8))
 (segment (start 174.65 84) (end 174.65 85.85) (width 0.6) (layer F.Cu) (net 12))
 (segment (start 173.04 87.46) (end 171.5 87.46) (width 0.6) (layer F.Cu) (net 12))
 (segment (start 174.65 85.85) (end 173.04 87.46) (width 0.6) (layer F.Cu) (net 12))
 (segment (start 157.15 77) (end 157.15 76.85) (width 0.6) (layer F.Cu) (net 2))
 (segment (start 157.45 76.55) (end 159.2 76.55) (width 0.6) (layer F.Cu) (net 2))
 (segment (start 157.15 76.85) (end 157.45 76.55) (width 0.6) (layer F.Cu) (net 2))
 (segment (start 160.55 76.55) (end 162 78) (width 0.6) (layer F.Cu) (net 2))
 (segment (start 159.2 76.55) (end 160.55 76.55) (width 0.6) (layer F.Cu) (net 2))
 (segment (start 154.95 98) (end 156.55 98) (width 0.6) (layer F.Cu) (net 5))
 (segment (start 159.2 79.45) (end 159.2 80.9) (width 0.6) (layer F.Cu) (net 7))
 (segment (start 160.3 82) (end 161.05 82) (width 0.6) (layer F.Cu) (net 7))
 (segment (start 159.2 80.9) (end 160.3 82) (width 0.6) (layer F.Cu) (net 7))
 (segment (start 152.65 77) (end 154.25 77) (width 0.6) (layer F.Cu) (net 4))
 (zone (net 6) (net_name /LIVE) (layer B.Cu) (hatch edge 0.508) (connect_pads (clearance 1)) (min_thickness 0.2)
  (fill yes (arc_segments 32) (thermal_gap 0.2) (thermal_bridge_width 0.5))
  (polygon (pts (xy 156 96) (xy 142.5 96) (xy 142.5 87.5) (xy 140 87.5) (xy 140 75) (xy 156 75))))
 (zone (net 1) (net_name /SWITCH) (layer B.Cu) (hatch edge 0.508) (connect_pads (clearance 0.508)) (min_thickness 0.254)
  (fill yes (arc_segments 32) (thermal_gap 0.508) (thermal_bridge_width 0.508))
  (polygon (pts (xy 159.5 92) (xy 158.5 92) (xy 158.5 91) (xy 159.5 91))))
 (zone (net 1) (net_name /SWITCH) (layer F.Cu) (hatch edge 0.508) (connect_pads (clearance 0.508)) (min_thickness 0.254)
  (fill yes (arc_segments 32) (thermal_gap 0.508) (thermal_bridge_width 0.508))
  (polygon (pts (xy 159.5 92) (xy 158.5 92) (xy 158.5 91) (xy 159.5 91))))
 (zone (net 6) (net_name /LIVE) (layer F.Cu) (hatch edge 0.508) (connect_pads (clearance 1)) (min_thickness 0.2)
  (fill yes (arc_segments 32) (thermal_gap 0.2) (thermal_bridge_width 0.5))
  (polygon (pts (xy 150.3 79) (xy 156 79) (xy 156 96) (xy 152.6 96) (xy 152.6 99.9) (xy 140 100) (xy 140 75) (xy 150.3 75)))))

